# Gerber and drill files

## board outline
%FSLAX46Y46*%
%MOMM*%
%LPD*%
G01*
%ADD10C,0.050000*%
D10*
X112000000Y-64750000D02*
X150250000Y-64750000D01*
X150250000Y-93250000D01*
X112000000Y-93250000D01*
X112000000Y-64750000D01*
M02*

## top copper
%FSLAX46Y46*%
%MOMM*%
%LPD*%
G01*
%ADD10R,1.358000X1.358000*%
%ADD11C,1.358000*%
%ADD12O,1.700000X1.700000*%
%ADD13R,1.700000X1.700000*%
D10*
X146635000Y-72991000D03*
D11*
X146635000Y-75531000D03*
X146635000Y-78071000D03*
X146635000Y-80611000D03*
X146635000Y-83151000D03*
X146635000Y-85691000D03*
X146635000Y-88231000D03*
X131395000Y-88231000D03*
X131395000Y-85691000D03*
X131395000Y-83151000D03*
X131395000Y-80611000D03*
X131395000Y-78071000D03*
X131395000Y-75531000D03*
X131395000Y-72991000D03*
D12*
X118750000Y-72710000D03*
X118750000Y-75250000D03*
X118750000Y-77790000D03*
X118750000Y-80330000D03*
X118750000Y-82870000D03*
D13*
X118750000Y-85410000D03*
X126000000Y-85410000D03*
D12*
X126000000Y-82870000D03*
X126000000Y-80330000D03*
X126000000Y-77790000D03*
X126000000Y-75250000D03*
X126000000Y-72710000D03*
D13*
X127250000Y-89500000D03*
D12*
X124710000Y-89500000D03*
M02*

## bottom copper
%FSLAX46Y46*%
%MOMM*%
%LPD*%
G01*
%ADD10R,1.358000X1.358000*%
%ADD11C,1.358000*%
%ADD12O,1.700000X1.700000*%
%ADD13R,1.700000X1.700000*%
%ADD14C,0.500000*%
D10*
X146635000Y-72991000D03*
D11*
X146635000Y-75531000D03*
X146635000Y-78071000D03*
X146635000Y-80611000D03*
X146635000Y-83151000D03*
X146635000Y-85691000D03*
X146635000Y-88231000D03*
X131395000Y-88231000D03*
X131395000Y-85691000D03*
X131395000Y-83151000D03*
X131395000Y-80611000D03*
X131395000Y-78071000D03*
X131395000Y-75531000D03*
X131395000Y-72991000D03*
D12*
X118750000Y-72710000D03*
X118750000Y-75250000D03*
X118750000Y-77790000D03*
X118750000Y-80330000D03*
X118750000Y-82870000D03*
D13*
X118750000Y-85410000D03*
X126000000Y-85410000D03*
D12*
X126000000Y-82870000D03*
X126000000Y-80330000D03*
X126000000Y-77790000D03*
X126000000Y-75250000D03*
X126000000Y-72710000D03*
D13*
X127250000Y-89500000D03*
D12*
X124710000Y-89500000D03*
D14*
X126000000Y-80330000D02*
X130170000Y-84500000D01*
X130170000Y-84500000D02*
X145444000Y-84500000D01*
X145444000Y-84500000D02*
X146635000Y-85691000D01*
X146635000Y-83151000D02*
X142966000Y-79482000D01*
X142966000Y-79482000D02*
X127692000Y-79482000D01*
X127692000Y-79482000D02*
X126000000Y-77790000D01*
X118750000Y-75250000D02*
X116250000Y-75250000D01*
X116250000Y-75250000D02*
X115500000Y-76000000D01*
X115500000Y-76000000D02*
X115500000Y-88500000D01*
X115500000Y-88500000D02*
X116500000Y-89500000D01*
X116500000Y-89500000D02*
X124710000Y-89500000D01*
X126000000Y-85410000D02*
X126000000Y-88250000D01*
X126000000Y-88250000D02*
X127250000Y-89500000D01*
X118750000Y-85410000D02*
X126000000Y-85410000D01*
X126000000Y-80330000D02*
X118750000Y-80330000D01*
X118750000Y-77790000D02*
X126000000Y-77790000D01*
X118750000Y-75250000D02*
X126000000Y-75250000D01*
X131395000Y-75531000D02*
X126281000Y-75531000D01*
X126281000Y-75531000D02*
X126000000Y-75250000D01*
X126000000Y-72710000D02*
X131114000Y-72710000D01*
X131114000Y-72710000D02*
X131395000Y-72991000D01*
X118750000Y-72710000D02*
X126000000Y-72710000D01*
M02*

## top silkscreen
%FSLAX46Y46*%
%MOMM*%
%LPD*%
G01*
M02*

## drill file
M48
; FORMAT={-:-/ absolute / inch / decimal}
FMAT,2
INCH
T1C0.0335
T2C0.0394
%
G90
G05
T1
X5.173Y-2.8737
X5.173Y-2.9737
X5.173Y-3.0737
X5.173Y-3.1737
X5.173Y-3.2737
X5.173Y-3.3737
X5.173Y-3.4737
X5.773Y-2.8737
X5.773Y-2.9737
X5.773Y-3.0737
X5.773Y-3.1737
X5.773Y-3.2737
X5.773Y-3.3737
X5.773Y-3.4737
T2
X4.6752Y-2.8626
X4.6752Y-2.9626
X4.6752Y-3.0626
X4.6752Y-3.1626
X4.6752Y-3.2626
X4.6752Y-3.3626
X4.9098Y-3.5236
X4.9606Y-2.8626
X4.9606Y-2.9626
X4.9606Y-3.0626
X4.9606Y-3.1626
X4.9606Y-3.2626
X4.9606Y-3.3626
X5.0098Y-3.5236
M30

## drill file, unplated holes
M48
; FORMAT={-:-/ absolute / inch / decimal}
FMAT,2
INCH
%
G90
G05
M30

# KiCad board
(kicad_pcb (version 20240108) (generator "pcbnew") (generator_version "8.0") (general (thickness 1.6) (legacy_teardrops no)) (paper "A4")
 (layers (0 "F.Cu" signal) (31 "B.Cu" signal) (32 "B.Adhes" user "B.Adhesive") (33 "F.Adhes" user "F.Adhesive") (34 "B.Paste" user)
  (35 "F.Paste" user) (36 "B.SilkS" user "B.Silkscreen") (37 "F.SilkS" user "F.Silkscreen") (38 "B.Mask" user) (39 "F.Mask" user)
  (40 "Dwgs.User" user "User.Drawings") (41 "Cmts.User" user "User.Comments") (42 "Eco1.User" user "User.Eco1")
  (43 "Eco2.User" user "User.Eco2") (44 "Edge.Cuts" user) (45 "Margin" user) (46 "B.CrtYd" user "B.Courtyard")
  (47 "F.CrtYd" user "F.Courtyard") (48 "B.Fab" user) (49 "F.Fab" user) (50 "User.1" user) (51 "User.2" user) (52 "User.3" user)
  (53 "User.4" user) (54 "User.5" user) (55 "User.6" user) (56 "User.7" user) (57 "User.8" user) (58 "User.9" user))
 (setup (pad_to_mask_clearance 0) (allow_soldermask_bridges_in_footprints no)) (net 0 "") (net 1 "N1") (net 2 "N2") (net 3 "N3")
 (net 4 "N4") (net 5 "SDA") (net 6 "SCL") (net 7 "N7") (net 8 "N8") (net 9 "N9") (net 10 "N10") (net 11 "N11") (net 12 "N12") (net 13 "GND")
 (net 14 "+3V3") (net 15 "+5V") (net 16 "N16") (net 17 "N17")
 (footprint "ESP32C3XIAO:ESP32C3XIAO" (layer "B.Cu") (at 139.015 80.5475 180)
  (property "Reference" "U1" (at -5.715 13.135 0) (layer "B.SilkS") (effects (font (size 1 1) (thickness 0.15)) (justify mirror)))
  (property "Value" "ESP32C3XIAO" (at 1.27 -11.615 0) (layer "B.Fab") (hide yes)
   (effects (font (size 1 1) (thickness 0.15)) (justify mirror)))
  (pad "1" thru_hole rect (at -7.62 7.5565 180) (size 1.358 1.358) (drill 0.85) (layers "*.Cu" "*.Mask") (remove_unused_layers no)
   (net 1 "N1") (solder_mask_margin 0.102))
  (pad "2" thru_hole circle (at -7.62 5.0165 180) (size 1.358 1.358) (drill 0.85) (layers "*.Cu" "*.Mask") (remove_unused_layers no)
   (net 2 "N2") (solder_mask_margin 0.102))
  (pad "3" thru_hole circle (at -7.62 2.4765 180) (size 1.358 1.358) (drill 0.85) (layers "*.Cu" "*.Mask") (remove_unused_layers no)
   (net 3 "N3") (solder_mask_margin 0.102))
  (pad "4" thru_hole circle (at -7.62 -0.0635 180) (size 1.358 1.358) (drill 0.85) (layers "*.Cu" "*.Mask") (remove_unused_layers no)
   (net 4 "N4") (solder_mask_margin 0.102))
  (pad "5" thru_hole circle (at -7.62 -2.6035 180) (size 1.358 1.358) (drill 0.85) (layers "*.Cu" "*.Mask") (remove_unused_layers no)
   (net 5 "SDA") (solder_mask_margin 0.102))
  (pad "6" thru_hole circle (at -7.62 -5.1435 180) (size 1.358 1.358) (drill 0.85) (layers "*.Cu" "*.Mask") (remove_unused_layers no)
   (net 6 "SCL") (solder_mask_margin 0.102))
  (pad "7" thru_hole circle (at -7.62 -7.6835 180) (size 1.358 1.358) (drill 0.85) (layers "*.Cu" "*.Mask") (remove_unused_layers no)
   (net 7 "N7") (solder_mask_margin 0.102))
  (pad "8" thru_hole circle (at 7.62 -7.6835 180) (size 1.358 1.358) (drill 0.85) (layers "*.Cu" "*.Mask") (remove_unused_layers no)
   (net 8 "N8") (solder_mask_margin 0.102))
  (pad "9" thru_hole circle (at 7.62 -5.1435 180) (size 1.358 1.358) (drill 0.85) (layers "*.Cu" "*.Mask") (remove_unused_layers no)
   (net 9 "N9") (solder_mask_margin 0.102))
  (pad "10" thru_hole circle (at 7.62 -2.6035 180) (size 1.358 1.358) (drill 0.85) (layers "*.Cu" "*.Mask") (remove_unused_layers no)
   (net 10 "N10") (solder_mask_margin 0.102))
  (pad "11" thru_hole circle (at 7.62 -0.0635 180) (size 1.358 1.358) (drill 0.85) (layers "*.Cu" "*.Mask") (remove_unused_layers no)
   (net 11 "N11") (solder_mask_margin 0.102))
  (pad "12" thru_hole circle (at 7.62 2.4765 180) (size 1.358 1.358) (drill 0.85) (layers "*.Cu" "*.Mask") (remove_unused_layers no)
   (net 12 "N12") (solder_mask_margin 0.102))
  (pad "13" thru_hole circle (at 7.62 5.0165 180) (size 1.358 1.358) (drill 0.85) (layers "*.Cu" "*.Mask") (remove_unused_layers no)
   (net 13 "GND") (solder_mask_margin 0.102))
  (pad "14" thru_hole circle (at 7.62 7.5565 180) (size 1.358 1.358) (drill 0.85) (layers "*.Cu" "*.Mask") (remove_unused_layers no)
   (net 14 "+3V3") (solder_mask_margin 0.102)))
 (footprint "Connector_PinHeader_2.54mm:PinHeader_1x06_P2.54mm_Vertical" (layer "B.Cu") (at 118.75 85.41)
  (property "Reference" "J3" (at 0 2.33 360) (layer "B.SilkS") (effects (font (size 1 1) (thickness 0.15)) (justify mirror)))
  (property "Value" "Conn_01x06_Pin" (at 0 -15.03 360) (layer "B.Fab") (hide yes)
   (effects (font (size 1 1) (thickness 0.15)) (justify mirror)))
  (pad "1" thru_hole rect (at 0 0) (size 1.7 1.7) (drill 1) (layers "*.Cu" "*.Mask") (remove_unused_layers no) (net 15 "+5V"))
  (pad "2" thru_hole oval (at 0 -2.54) (size 1.7 1.7) (drill 1) (layers "*.Cu" "*.Mask") (remove_unused_layers no) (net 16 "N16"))
  (pad "3" thru_hole oval (at 0 -5.08) (size 1.7 1.7) (drill 1) (layers "*.Cu" "*.Mask") (remove_unused_layers no) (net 6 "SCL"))
  (pad "4" thru_hole oval (at 0 -7.62) (size 1.7 1.7) (drill 1) (layers "*.Cu" "*.Mask") (remove_unused_layers no) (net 5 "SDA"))
  (pad "5" thru_hole oval (at 0 -10.16) (size 1.7 1.7) (drill 1) (layers "*.Cu" "*.Mask") (remove_unused_layers no) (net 13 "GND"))
  (pad "6" thru_hole oval (at 0 -12.7) (size 1.7 1.7) (drill 1) (layers "*.Cu" "*.Mask") (remove_unused_layers no) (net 14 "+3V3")))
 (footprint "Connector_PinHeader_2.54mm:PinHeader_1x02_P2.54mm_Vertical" (layer "B.Cu") (at 127.25 89.5 90)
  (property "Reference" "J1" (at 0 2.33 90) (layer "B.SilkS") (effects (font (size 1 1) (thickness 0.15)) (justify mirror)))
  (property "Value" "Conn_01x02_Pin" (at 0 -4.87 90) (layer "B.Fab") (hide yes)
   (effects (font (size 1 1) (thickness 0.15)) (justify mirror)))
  (pad "1" thru_hole rect (at 0 0 90) (size 1.7 1.7) (drill 1) (layers "*.Cu" "*.Mask") (remove_unused_layers no) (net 15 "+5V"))
  (pad "2" thru_hole oval (at 0 -2.54 90) (size 1.7 1.7) (drill 1) (layers "*.Cu" "*.Mask") (remove_unused_layers no) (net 13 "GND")))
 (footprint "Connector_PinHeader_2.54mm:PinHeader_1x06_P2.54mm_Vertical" (layer "B.Cu") (at 126 85.41)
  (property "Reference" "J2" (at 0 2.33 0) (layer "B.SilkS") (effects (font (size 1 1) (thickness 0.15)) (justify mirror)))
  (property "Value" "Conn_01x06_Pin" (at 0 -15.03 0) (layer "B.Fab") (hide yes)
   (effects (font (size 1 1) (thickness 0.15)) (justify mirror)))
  (pad "1" thru_hole rect (at 0 0) (size 1.7 1.7) (drill 1) (layers "*.Cu" "*.Mask") (remove_unused_layers no) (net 15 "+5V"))
  (pad "2" thru_hole oval (at 0 -2.54) (size 1.7 1.7) (drill 1) (layers "*.Cu" "*.Mask") (remove_unused_layers no) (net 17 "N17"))
  (pad "3" thru_hole oval (at 0 -5.08) (size 1.7 1.7) (drill 1) (layers "*.Cu" "*.Mask") (remove_unused_layers no) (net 6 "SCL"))
  (pad "4" thru_hole oval (at 0 -7.62) (size 1.7 1.7) (drill 1) (layers "*.Cu" "*.Mask") (remove_unused_layers no) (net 5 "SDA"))
  (pad "5" thru_hole oval (at 0 -10.16) (size 1.7 1.7) (drill 1) (layers "*.Cu" "*.Mask") (remove_unused_layers no) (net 13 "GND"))
  (pad "6" thru_hole oval (at 0 -12.7) (size 1.7 1.7) (drill 1) (layers "*.Cu" "*.Mask") (remove_unused_layers no) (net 14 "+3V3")))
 (gr_rect (start 112 64.75) (end 150.25 93.25) (stroke (width 0.05) (type default)) (fill none) (layer "Edge.Cuts"))
 (segment (start 116.25 75.25) (end 115.5 76) (width 0.5) (layer "B.Cu") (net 13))
 (segment (start 118.75 75.25) (end 126 75.25) (width 0.5) (layer "B.Cu") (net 13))
 (segment (start 126.281 75.531) (end 126 75.25) (width 0.5) (layer "B.Cu") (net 13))
 (segment (start 116.5 89.5) (end 124.71 89.5) (width 0.5) (layer "B.Cu") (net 13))
 (segment (start 131.395 75.531) (end 126.281 75.531) (width 0.5) (layer "B.Cu") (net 13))
 (segment (start 115.5 76) (end 115.5 88.5) (width 0.5) (layer "B.Cu") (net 13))
 (segment (start 118.75 75.25) (end 116.25 75.25) (width 0.5) (layer "B.Cu") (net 13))
 (segment (start 115.5 88.5) (end 116.5 89.5) (width 0.5) (layer "B.Cu") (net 13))
 (segment (start 126 88.25) (end 127.25 89.5) (width 0.5) (layer "B.Cu") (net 15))
 (segment (start 118.75 85.41) (end 126 85.41) (width 0.5) (layer "B.Cu") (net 15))
 (segment (start 126 85.41) (end 126 88.25) (width 0.5) (layer "B.Cu") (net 15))
 (segment (start 142.966 79.482) (end 127.692 79.482) (width 0.5) (layer "B.Cu") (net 5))
 (segment (start 118.75 77.79) (end 126 77.79) (width 0.5) (layer "B.Cu") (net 5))
 (segment (start 146.635 83.151) (end 142.966 79.482) (width 0.5) (layer "B.Cu") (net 5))
 (segment (start 127.692 79.482) (end 126 77.79) (width 0.5) (layer "B.Cu") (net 5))
 (segment (start 126 80.33) (end 118.75 80.33) (width 0.5) (layer "B.Cu") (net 6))
 (segment (start 130.17 84.5) (end 145.444 84.5) (width 0.5) (layer "B.Cu") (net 6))
 (segment (start 145.444 84.5) (end 146.635 85.691) (width 0.5) (layer "B.Cu") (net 6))
 (segment (start 126 80.33) (end 130.17 84.5) (width 0.5) (layer "B.Cu") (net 6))
 (segment (start 118.75 72.71) (end 126 72.71) (width 0.5) (layer "B.Cu") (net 14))
 (segment (start 131.114 72.71) (end 131.395 72.991) (width 0.5) (layer "B.Cu") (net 14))
 (segment (start 126 72.71) (end 131.114 72.71) (width 0.5) (layer "B.Cu") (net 14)))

